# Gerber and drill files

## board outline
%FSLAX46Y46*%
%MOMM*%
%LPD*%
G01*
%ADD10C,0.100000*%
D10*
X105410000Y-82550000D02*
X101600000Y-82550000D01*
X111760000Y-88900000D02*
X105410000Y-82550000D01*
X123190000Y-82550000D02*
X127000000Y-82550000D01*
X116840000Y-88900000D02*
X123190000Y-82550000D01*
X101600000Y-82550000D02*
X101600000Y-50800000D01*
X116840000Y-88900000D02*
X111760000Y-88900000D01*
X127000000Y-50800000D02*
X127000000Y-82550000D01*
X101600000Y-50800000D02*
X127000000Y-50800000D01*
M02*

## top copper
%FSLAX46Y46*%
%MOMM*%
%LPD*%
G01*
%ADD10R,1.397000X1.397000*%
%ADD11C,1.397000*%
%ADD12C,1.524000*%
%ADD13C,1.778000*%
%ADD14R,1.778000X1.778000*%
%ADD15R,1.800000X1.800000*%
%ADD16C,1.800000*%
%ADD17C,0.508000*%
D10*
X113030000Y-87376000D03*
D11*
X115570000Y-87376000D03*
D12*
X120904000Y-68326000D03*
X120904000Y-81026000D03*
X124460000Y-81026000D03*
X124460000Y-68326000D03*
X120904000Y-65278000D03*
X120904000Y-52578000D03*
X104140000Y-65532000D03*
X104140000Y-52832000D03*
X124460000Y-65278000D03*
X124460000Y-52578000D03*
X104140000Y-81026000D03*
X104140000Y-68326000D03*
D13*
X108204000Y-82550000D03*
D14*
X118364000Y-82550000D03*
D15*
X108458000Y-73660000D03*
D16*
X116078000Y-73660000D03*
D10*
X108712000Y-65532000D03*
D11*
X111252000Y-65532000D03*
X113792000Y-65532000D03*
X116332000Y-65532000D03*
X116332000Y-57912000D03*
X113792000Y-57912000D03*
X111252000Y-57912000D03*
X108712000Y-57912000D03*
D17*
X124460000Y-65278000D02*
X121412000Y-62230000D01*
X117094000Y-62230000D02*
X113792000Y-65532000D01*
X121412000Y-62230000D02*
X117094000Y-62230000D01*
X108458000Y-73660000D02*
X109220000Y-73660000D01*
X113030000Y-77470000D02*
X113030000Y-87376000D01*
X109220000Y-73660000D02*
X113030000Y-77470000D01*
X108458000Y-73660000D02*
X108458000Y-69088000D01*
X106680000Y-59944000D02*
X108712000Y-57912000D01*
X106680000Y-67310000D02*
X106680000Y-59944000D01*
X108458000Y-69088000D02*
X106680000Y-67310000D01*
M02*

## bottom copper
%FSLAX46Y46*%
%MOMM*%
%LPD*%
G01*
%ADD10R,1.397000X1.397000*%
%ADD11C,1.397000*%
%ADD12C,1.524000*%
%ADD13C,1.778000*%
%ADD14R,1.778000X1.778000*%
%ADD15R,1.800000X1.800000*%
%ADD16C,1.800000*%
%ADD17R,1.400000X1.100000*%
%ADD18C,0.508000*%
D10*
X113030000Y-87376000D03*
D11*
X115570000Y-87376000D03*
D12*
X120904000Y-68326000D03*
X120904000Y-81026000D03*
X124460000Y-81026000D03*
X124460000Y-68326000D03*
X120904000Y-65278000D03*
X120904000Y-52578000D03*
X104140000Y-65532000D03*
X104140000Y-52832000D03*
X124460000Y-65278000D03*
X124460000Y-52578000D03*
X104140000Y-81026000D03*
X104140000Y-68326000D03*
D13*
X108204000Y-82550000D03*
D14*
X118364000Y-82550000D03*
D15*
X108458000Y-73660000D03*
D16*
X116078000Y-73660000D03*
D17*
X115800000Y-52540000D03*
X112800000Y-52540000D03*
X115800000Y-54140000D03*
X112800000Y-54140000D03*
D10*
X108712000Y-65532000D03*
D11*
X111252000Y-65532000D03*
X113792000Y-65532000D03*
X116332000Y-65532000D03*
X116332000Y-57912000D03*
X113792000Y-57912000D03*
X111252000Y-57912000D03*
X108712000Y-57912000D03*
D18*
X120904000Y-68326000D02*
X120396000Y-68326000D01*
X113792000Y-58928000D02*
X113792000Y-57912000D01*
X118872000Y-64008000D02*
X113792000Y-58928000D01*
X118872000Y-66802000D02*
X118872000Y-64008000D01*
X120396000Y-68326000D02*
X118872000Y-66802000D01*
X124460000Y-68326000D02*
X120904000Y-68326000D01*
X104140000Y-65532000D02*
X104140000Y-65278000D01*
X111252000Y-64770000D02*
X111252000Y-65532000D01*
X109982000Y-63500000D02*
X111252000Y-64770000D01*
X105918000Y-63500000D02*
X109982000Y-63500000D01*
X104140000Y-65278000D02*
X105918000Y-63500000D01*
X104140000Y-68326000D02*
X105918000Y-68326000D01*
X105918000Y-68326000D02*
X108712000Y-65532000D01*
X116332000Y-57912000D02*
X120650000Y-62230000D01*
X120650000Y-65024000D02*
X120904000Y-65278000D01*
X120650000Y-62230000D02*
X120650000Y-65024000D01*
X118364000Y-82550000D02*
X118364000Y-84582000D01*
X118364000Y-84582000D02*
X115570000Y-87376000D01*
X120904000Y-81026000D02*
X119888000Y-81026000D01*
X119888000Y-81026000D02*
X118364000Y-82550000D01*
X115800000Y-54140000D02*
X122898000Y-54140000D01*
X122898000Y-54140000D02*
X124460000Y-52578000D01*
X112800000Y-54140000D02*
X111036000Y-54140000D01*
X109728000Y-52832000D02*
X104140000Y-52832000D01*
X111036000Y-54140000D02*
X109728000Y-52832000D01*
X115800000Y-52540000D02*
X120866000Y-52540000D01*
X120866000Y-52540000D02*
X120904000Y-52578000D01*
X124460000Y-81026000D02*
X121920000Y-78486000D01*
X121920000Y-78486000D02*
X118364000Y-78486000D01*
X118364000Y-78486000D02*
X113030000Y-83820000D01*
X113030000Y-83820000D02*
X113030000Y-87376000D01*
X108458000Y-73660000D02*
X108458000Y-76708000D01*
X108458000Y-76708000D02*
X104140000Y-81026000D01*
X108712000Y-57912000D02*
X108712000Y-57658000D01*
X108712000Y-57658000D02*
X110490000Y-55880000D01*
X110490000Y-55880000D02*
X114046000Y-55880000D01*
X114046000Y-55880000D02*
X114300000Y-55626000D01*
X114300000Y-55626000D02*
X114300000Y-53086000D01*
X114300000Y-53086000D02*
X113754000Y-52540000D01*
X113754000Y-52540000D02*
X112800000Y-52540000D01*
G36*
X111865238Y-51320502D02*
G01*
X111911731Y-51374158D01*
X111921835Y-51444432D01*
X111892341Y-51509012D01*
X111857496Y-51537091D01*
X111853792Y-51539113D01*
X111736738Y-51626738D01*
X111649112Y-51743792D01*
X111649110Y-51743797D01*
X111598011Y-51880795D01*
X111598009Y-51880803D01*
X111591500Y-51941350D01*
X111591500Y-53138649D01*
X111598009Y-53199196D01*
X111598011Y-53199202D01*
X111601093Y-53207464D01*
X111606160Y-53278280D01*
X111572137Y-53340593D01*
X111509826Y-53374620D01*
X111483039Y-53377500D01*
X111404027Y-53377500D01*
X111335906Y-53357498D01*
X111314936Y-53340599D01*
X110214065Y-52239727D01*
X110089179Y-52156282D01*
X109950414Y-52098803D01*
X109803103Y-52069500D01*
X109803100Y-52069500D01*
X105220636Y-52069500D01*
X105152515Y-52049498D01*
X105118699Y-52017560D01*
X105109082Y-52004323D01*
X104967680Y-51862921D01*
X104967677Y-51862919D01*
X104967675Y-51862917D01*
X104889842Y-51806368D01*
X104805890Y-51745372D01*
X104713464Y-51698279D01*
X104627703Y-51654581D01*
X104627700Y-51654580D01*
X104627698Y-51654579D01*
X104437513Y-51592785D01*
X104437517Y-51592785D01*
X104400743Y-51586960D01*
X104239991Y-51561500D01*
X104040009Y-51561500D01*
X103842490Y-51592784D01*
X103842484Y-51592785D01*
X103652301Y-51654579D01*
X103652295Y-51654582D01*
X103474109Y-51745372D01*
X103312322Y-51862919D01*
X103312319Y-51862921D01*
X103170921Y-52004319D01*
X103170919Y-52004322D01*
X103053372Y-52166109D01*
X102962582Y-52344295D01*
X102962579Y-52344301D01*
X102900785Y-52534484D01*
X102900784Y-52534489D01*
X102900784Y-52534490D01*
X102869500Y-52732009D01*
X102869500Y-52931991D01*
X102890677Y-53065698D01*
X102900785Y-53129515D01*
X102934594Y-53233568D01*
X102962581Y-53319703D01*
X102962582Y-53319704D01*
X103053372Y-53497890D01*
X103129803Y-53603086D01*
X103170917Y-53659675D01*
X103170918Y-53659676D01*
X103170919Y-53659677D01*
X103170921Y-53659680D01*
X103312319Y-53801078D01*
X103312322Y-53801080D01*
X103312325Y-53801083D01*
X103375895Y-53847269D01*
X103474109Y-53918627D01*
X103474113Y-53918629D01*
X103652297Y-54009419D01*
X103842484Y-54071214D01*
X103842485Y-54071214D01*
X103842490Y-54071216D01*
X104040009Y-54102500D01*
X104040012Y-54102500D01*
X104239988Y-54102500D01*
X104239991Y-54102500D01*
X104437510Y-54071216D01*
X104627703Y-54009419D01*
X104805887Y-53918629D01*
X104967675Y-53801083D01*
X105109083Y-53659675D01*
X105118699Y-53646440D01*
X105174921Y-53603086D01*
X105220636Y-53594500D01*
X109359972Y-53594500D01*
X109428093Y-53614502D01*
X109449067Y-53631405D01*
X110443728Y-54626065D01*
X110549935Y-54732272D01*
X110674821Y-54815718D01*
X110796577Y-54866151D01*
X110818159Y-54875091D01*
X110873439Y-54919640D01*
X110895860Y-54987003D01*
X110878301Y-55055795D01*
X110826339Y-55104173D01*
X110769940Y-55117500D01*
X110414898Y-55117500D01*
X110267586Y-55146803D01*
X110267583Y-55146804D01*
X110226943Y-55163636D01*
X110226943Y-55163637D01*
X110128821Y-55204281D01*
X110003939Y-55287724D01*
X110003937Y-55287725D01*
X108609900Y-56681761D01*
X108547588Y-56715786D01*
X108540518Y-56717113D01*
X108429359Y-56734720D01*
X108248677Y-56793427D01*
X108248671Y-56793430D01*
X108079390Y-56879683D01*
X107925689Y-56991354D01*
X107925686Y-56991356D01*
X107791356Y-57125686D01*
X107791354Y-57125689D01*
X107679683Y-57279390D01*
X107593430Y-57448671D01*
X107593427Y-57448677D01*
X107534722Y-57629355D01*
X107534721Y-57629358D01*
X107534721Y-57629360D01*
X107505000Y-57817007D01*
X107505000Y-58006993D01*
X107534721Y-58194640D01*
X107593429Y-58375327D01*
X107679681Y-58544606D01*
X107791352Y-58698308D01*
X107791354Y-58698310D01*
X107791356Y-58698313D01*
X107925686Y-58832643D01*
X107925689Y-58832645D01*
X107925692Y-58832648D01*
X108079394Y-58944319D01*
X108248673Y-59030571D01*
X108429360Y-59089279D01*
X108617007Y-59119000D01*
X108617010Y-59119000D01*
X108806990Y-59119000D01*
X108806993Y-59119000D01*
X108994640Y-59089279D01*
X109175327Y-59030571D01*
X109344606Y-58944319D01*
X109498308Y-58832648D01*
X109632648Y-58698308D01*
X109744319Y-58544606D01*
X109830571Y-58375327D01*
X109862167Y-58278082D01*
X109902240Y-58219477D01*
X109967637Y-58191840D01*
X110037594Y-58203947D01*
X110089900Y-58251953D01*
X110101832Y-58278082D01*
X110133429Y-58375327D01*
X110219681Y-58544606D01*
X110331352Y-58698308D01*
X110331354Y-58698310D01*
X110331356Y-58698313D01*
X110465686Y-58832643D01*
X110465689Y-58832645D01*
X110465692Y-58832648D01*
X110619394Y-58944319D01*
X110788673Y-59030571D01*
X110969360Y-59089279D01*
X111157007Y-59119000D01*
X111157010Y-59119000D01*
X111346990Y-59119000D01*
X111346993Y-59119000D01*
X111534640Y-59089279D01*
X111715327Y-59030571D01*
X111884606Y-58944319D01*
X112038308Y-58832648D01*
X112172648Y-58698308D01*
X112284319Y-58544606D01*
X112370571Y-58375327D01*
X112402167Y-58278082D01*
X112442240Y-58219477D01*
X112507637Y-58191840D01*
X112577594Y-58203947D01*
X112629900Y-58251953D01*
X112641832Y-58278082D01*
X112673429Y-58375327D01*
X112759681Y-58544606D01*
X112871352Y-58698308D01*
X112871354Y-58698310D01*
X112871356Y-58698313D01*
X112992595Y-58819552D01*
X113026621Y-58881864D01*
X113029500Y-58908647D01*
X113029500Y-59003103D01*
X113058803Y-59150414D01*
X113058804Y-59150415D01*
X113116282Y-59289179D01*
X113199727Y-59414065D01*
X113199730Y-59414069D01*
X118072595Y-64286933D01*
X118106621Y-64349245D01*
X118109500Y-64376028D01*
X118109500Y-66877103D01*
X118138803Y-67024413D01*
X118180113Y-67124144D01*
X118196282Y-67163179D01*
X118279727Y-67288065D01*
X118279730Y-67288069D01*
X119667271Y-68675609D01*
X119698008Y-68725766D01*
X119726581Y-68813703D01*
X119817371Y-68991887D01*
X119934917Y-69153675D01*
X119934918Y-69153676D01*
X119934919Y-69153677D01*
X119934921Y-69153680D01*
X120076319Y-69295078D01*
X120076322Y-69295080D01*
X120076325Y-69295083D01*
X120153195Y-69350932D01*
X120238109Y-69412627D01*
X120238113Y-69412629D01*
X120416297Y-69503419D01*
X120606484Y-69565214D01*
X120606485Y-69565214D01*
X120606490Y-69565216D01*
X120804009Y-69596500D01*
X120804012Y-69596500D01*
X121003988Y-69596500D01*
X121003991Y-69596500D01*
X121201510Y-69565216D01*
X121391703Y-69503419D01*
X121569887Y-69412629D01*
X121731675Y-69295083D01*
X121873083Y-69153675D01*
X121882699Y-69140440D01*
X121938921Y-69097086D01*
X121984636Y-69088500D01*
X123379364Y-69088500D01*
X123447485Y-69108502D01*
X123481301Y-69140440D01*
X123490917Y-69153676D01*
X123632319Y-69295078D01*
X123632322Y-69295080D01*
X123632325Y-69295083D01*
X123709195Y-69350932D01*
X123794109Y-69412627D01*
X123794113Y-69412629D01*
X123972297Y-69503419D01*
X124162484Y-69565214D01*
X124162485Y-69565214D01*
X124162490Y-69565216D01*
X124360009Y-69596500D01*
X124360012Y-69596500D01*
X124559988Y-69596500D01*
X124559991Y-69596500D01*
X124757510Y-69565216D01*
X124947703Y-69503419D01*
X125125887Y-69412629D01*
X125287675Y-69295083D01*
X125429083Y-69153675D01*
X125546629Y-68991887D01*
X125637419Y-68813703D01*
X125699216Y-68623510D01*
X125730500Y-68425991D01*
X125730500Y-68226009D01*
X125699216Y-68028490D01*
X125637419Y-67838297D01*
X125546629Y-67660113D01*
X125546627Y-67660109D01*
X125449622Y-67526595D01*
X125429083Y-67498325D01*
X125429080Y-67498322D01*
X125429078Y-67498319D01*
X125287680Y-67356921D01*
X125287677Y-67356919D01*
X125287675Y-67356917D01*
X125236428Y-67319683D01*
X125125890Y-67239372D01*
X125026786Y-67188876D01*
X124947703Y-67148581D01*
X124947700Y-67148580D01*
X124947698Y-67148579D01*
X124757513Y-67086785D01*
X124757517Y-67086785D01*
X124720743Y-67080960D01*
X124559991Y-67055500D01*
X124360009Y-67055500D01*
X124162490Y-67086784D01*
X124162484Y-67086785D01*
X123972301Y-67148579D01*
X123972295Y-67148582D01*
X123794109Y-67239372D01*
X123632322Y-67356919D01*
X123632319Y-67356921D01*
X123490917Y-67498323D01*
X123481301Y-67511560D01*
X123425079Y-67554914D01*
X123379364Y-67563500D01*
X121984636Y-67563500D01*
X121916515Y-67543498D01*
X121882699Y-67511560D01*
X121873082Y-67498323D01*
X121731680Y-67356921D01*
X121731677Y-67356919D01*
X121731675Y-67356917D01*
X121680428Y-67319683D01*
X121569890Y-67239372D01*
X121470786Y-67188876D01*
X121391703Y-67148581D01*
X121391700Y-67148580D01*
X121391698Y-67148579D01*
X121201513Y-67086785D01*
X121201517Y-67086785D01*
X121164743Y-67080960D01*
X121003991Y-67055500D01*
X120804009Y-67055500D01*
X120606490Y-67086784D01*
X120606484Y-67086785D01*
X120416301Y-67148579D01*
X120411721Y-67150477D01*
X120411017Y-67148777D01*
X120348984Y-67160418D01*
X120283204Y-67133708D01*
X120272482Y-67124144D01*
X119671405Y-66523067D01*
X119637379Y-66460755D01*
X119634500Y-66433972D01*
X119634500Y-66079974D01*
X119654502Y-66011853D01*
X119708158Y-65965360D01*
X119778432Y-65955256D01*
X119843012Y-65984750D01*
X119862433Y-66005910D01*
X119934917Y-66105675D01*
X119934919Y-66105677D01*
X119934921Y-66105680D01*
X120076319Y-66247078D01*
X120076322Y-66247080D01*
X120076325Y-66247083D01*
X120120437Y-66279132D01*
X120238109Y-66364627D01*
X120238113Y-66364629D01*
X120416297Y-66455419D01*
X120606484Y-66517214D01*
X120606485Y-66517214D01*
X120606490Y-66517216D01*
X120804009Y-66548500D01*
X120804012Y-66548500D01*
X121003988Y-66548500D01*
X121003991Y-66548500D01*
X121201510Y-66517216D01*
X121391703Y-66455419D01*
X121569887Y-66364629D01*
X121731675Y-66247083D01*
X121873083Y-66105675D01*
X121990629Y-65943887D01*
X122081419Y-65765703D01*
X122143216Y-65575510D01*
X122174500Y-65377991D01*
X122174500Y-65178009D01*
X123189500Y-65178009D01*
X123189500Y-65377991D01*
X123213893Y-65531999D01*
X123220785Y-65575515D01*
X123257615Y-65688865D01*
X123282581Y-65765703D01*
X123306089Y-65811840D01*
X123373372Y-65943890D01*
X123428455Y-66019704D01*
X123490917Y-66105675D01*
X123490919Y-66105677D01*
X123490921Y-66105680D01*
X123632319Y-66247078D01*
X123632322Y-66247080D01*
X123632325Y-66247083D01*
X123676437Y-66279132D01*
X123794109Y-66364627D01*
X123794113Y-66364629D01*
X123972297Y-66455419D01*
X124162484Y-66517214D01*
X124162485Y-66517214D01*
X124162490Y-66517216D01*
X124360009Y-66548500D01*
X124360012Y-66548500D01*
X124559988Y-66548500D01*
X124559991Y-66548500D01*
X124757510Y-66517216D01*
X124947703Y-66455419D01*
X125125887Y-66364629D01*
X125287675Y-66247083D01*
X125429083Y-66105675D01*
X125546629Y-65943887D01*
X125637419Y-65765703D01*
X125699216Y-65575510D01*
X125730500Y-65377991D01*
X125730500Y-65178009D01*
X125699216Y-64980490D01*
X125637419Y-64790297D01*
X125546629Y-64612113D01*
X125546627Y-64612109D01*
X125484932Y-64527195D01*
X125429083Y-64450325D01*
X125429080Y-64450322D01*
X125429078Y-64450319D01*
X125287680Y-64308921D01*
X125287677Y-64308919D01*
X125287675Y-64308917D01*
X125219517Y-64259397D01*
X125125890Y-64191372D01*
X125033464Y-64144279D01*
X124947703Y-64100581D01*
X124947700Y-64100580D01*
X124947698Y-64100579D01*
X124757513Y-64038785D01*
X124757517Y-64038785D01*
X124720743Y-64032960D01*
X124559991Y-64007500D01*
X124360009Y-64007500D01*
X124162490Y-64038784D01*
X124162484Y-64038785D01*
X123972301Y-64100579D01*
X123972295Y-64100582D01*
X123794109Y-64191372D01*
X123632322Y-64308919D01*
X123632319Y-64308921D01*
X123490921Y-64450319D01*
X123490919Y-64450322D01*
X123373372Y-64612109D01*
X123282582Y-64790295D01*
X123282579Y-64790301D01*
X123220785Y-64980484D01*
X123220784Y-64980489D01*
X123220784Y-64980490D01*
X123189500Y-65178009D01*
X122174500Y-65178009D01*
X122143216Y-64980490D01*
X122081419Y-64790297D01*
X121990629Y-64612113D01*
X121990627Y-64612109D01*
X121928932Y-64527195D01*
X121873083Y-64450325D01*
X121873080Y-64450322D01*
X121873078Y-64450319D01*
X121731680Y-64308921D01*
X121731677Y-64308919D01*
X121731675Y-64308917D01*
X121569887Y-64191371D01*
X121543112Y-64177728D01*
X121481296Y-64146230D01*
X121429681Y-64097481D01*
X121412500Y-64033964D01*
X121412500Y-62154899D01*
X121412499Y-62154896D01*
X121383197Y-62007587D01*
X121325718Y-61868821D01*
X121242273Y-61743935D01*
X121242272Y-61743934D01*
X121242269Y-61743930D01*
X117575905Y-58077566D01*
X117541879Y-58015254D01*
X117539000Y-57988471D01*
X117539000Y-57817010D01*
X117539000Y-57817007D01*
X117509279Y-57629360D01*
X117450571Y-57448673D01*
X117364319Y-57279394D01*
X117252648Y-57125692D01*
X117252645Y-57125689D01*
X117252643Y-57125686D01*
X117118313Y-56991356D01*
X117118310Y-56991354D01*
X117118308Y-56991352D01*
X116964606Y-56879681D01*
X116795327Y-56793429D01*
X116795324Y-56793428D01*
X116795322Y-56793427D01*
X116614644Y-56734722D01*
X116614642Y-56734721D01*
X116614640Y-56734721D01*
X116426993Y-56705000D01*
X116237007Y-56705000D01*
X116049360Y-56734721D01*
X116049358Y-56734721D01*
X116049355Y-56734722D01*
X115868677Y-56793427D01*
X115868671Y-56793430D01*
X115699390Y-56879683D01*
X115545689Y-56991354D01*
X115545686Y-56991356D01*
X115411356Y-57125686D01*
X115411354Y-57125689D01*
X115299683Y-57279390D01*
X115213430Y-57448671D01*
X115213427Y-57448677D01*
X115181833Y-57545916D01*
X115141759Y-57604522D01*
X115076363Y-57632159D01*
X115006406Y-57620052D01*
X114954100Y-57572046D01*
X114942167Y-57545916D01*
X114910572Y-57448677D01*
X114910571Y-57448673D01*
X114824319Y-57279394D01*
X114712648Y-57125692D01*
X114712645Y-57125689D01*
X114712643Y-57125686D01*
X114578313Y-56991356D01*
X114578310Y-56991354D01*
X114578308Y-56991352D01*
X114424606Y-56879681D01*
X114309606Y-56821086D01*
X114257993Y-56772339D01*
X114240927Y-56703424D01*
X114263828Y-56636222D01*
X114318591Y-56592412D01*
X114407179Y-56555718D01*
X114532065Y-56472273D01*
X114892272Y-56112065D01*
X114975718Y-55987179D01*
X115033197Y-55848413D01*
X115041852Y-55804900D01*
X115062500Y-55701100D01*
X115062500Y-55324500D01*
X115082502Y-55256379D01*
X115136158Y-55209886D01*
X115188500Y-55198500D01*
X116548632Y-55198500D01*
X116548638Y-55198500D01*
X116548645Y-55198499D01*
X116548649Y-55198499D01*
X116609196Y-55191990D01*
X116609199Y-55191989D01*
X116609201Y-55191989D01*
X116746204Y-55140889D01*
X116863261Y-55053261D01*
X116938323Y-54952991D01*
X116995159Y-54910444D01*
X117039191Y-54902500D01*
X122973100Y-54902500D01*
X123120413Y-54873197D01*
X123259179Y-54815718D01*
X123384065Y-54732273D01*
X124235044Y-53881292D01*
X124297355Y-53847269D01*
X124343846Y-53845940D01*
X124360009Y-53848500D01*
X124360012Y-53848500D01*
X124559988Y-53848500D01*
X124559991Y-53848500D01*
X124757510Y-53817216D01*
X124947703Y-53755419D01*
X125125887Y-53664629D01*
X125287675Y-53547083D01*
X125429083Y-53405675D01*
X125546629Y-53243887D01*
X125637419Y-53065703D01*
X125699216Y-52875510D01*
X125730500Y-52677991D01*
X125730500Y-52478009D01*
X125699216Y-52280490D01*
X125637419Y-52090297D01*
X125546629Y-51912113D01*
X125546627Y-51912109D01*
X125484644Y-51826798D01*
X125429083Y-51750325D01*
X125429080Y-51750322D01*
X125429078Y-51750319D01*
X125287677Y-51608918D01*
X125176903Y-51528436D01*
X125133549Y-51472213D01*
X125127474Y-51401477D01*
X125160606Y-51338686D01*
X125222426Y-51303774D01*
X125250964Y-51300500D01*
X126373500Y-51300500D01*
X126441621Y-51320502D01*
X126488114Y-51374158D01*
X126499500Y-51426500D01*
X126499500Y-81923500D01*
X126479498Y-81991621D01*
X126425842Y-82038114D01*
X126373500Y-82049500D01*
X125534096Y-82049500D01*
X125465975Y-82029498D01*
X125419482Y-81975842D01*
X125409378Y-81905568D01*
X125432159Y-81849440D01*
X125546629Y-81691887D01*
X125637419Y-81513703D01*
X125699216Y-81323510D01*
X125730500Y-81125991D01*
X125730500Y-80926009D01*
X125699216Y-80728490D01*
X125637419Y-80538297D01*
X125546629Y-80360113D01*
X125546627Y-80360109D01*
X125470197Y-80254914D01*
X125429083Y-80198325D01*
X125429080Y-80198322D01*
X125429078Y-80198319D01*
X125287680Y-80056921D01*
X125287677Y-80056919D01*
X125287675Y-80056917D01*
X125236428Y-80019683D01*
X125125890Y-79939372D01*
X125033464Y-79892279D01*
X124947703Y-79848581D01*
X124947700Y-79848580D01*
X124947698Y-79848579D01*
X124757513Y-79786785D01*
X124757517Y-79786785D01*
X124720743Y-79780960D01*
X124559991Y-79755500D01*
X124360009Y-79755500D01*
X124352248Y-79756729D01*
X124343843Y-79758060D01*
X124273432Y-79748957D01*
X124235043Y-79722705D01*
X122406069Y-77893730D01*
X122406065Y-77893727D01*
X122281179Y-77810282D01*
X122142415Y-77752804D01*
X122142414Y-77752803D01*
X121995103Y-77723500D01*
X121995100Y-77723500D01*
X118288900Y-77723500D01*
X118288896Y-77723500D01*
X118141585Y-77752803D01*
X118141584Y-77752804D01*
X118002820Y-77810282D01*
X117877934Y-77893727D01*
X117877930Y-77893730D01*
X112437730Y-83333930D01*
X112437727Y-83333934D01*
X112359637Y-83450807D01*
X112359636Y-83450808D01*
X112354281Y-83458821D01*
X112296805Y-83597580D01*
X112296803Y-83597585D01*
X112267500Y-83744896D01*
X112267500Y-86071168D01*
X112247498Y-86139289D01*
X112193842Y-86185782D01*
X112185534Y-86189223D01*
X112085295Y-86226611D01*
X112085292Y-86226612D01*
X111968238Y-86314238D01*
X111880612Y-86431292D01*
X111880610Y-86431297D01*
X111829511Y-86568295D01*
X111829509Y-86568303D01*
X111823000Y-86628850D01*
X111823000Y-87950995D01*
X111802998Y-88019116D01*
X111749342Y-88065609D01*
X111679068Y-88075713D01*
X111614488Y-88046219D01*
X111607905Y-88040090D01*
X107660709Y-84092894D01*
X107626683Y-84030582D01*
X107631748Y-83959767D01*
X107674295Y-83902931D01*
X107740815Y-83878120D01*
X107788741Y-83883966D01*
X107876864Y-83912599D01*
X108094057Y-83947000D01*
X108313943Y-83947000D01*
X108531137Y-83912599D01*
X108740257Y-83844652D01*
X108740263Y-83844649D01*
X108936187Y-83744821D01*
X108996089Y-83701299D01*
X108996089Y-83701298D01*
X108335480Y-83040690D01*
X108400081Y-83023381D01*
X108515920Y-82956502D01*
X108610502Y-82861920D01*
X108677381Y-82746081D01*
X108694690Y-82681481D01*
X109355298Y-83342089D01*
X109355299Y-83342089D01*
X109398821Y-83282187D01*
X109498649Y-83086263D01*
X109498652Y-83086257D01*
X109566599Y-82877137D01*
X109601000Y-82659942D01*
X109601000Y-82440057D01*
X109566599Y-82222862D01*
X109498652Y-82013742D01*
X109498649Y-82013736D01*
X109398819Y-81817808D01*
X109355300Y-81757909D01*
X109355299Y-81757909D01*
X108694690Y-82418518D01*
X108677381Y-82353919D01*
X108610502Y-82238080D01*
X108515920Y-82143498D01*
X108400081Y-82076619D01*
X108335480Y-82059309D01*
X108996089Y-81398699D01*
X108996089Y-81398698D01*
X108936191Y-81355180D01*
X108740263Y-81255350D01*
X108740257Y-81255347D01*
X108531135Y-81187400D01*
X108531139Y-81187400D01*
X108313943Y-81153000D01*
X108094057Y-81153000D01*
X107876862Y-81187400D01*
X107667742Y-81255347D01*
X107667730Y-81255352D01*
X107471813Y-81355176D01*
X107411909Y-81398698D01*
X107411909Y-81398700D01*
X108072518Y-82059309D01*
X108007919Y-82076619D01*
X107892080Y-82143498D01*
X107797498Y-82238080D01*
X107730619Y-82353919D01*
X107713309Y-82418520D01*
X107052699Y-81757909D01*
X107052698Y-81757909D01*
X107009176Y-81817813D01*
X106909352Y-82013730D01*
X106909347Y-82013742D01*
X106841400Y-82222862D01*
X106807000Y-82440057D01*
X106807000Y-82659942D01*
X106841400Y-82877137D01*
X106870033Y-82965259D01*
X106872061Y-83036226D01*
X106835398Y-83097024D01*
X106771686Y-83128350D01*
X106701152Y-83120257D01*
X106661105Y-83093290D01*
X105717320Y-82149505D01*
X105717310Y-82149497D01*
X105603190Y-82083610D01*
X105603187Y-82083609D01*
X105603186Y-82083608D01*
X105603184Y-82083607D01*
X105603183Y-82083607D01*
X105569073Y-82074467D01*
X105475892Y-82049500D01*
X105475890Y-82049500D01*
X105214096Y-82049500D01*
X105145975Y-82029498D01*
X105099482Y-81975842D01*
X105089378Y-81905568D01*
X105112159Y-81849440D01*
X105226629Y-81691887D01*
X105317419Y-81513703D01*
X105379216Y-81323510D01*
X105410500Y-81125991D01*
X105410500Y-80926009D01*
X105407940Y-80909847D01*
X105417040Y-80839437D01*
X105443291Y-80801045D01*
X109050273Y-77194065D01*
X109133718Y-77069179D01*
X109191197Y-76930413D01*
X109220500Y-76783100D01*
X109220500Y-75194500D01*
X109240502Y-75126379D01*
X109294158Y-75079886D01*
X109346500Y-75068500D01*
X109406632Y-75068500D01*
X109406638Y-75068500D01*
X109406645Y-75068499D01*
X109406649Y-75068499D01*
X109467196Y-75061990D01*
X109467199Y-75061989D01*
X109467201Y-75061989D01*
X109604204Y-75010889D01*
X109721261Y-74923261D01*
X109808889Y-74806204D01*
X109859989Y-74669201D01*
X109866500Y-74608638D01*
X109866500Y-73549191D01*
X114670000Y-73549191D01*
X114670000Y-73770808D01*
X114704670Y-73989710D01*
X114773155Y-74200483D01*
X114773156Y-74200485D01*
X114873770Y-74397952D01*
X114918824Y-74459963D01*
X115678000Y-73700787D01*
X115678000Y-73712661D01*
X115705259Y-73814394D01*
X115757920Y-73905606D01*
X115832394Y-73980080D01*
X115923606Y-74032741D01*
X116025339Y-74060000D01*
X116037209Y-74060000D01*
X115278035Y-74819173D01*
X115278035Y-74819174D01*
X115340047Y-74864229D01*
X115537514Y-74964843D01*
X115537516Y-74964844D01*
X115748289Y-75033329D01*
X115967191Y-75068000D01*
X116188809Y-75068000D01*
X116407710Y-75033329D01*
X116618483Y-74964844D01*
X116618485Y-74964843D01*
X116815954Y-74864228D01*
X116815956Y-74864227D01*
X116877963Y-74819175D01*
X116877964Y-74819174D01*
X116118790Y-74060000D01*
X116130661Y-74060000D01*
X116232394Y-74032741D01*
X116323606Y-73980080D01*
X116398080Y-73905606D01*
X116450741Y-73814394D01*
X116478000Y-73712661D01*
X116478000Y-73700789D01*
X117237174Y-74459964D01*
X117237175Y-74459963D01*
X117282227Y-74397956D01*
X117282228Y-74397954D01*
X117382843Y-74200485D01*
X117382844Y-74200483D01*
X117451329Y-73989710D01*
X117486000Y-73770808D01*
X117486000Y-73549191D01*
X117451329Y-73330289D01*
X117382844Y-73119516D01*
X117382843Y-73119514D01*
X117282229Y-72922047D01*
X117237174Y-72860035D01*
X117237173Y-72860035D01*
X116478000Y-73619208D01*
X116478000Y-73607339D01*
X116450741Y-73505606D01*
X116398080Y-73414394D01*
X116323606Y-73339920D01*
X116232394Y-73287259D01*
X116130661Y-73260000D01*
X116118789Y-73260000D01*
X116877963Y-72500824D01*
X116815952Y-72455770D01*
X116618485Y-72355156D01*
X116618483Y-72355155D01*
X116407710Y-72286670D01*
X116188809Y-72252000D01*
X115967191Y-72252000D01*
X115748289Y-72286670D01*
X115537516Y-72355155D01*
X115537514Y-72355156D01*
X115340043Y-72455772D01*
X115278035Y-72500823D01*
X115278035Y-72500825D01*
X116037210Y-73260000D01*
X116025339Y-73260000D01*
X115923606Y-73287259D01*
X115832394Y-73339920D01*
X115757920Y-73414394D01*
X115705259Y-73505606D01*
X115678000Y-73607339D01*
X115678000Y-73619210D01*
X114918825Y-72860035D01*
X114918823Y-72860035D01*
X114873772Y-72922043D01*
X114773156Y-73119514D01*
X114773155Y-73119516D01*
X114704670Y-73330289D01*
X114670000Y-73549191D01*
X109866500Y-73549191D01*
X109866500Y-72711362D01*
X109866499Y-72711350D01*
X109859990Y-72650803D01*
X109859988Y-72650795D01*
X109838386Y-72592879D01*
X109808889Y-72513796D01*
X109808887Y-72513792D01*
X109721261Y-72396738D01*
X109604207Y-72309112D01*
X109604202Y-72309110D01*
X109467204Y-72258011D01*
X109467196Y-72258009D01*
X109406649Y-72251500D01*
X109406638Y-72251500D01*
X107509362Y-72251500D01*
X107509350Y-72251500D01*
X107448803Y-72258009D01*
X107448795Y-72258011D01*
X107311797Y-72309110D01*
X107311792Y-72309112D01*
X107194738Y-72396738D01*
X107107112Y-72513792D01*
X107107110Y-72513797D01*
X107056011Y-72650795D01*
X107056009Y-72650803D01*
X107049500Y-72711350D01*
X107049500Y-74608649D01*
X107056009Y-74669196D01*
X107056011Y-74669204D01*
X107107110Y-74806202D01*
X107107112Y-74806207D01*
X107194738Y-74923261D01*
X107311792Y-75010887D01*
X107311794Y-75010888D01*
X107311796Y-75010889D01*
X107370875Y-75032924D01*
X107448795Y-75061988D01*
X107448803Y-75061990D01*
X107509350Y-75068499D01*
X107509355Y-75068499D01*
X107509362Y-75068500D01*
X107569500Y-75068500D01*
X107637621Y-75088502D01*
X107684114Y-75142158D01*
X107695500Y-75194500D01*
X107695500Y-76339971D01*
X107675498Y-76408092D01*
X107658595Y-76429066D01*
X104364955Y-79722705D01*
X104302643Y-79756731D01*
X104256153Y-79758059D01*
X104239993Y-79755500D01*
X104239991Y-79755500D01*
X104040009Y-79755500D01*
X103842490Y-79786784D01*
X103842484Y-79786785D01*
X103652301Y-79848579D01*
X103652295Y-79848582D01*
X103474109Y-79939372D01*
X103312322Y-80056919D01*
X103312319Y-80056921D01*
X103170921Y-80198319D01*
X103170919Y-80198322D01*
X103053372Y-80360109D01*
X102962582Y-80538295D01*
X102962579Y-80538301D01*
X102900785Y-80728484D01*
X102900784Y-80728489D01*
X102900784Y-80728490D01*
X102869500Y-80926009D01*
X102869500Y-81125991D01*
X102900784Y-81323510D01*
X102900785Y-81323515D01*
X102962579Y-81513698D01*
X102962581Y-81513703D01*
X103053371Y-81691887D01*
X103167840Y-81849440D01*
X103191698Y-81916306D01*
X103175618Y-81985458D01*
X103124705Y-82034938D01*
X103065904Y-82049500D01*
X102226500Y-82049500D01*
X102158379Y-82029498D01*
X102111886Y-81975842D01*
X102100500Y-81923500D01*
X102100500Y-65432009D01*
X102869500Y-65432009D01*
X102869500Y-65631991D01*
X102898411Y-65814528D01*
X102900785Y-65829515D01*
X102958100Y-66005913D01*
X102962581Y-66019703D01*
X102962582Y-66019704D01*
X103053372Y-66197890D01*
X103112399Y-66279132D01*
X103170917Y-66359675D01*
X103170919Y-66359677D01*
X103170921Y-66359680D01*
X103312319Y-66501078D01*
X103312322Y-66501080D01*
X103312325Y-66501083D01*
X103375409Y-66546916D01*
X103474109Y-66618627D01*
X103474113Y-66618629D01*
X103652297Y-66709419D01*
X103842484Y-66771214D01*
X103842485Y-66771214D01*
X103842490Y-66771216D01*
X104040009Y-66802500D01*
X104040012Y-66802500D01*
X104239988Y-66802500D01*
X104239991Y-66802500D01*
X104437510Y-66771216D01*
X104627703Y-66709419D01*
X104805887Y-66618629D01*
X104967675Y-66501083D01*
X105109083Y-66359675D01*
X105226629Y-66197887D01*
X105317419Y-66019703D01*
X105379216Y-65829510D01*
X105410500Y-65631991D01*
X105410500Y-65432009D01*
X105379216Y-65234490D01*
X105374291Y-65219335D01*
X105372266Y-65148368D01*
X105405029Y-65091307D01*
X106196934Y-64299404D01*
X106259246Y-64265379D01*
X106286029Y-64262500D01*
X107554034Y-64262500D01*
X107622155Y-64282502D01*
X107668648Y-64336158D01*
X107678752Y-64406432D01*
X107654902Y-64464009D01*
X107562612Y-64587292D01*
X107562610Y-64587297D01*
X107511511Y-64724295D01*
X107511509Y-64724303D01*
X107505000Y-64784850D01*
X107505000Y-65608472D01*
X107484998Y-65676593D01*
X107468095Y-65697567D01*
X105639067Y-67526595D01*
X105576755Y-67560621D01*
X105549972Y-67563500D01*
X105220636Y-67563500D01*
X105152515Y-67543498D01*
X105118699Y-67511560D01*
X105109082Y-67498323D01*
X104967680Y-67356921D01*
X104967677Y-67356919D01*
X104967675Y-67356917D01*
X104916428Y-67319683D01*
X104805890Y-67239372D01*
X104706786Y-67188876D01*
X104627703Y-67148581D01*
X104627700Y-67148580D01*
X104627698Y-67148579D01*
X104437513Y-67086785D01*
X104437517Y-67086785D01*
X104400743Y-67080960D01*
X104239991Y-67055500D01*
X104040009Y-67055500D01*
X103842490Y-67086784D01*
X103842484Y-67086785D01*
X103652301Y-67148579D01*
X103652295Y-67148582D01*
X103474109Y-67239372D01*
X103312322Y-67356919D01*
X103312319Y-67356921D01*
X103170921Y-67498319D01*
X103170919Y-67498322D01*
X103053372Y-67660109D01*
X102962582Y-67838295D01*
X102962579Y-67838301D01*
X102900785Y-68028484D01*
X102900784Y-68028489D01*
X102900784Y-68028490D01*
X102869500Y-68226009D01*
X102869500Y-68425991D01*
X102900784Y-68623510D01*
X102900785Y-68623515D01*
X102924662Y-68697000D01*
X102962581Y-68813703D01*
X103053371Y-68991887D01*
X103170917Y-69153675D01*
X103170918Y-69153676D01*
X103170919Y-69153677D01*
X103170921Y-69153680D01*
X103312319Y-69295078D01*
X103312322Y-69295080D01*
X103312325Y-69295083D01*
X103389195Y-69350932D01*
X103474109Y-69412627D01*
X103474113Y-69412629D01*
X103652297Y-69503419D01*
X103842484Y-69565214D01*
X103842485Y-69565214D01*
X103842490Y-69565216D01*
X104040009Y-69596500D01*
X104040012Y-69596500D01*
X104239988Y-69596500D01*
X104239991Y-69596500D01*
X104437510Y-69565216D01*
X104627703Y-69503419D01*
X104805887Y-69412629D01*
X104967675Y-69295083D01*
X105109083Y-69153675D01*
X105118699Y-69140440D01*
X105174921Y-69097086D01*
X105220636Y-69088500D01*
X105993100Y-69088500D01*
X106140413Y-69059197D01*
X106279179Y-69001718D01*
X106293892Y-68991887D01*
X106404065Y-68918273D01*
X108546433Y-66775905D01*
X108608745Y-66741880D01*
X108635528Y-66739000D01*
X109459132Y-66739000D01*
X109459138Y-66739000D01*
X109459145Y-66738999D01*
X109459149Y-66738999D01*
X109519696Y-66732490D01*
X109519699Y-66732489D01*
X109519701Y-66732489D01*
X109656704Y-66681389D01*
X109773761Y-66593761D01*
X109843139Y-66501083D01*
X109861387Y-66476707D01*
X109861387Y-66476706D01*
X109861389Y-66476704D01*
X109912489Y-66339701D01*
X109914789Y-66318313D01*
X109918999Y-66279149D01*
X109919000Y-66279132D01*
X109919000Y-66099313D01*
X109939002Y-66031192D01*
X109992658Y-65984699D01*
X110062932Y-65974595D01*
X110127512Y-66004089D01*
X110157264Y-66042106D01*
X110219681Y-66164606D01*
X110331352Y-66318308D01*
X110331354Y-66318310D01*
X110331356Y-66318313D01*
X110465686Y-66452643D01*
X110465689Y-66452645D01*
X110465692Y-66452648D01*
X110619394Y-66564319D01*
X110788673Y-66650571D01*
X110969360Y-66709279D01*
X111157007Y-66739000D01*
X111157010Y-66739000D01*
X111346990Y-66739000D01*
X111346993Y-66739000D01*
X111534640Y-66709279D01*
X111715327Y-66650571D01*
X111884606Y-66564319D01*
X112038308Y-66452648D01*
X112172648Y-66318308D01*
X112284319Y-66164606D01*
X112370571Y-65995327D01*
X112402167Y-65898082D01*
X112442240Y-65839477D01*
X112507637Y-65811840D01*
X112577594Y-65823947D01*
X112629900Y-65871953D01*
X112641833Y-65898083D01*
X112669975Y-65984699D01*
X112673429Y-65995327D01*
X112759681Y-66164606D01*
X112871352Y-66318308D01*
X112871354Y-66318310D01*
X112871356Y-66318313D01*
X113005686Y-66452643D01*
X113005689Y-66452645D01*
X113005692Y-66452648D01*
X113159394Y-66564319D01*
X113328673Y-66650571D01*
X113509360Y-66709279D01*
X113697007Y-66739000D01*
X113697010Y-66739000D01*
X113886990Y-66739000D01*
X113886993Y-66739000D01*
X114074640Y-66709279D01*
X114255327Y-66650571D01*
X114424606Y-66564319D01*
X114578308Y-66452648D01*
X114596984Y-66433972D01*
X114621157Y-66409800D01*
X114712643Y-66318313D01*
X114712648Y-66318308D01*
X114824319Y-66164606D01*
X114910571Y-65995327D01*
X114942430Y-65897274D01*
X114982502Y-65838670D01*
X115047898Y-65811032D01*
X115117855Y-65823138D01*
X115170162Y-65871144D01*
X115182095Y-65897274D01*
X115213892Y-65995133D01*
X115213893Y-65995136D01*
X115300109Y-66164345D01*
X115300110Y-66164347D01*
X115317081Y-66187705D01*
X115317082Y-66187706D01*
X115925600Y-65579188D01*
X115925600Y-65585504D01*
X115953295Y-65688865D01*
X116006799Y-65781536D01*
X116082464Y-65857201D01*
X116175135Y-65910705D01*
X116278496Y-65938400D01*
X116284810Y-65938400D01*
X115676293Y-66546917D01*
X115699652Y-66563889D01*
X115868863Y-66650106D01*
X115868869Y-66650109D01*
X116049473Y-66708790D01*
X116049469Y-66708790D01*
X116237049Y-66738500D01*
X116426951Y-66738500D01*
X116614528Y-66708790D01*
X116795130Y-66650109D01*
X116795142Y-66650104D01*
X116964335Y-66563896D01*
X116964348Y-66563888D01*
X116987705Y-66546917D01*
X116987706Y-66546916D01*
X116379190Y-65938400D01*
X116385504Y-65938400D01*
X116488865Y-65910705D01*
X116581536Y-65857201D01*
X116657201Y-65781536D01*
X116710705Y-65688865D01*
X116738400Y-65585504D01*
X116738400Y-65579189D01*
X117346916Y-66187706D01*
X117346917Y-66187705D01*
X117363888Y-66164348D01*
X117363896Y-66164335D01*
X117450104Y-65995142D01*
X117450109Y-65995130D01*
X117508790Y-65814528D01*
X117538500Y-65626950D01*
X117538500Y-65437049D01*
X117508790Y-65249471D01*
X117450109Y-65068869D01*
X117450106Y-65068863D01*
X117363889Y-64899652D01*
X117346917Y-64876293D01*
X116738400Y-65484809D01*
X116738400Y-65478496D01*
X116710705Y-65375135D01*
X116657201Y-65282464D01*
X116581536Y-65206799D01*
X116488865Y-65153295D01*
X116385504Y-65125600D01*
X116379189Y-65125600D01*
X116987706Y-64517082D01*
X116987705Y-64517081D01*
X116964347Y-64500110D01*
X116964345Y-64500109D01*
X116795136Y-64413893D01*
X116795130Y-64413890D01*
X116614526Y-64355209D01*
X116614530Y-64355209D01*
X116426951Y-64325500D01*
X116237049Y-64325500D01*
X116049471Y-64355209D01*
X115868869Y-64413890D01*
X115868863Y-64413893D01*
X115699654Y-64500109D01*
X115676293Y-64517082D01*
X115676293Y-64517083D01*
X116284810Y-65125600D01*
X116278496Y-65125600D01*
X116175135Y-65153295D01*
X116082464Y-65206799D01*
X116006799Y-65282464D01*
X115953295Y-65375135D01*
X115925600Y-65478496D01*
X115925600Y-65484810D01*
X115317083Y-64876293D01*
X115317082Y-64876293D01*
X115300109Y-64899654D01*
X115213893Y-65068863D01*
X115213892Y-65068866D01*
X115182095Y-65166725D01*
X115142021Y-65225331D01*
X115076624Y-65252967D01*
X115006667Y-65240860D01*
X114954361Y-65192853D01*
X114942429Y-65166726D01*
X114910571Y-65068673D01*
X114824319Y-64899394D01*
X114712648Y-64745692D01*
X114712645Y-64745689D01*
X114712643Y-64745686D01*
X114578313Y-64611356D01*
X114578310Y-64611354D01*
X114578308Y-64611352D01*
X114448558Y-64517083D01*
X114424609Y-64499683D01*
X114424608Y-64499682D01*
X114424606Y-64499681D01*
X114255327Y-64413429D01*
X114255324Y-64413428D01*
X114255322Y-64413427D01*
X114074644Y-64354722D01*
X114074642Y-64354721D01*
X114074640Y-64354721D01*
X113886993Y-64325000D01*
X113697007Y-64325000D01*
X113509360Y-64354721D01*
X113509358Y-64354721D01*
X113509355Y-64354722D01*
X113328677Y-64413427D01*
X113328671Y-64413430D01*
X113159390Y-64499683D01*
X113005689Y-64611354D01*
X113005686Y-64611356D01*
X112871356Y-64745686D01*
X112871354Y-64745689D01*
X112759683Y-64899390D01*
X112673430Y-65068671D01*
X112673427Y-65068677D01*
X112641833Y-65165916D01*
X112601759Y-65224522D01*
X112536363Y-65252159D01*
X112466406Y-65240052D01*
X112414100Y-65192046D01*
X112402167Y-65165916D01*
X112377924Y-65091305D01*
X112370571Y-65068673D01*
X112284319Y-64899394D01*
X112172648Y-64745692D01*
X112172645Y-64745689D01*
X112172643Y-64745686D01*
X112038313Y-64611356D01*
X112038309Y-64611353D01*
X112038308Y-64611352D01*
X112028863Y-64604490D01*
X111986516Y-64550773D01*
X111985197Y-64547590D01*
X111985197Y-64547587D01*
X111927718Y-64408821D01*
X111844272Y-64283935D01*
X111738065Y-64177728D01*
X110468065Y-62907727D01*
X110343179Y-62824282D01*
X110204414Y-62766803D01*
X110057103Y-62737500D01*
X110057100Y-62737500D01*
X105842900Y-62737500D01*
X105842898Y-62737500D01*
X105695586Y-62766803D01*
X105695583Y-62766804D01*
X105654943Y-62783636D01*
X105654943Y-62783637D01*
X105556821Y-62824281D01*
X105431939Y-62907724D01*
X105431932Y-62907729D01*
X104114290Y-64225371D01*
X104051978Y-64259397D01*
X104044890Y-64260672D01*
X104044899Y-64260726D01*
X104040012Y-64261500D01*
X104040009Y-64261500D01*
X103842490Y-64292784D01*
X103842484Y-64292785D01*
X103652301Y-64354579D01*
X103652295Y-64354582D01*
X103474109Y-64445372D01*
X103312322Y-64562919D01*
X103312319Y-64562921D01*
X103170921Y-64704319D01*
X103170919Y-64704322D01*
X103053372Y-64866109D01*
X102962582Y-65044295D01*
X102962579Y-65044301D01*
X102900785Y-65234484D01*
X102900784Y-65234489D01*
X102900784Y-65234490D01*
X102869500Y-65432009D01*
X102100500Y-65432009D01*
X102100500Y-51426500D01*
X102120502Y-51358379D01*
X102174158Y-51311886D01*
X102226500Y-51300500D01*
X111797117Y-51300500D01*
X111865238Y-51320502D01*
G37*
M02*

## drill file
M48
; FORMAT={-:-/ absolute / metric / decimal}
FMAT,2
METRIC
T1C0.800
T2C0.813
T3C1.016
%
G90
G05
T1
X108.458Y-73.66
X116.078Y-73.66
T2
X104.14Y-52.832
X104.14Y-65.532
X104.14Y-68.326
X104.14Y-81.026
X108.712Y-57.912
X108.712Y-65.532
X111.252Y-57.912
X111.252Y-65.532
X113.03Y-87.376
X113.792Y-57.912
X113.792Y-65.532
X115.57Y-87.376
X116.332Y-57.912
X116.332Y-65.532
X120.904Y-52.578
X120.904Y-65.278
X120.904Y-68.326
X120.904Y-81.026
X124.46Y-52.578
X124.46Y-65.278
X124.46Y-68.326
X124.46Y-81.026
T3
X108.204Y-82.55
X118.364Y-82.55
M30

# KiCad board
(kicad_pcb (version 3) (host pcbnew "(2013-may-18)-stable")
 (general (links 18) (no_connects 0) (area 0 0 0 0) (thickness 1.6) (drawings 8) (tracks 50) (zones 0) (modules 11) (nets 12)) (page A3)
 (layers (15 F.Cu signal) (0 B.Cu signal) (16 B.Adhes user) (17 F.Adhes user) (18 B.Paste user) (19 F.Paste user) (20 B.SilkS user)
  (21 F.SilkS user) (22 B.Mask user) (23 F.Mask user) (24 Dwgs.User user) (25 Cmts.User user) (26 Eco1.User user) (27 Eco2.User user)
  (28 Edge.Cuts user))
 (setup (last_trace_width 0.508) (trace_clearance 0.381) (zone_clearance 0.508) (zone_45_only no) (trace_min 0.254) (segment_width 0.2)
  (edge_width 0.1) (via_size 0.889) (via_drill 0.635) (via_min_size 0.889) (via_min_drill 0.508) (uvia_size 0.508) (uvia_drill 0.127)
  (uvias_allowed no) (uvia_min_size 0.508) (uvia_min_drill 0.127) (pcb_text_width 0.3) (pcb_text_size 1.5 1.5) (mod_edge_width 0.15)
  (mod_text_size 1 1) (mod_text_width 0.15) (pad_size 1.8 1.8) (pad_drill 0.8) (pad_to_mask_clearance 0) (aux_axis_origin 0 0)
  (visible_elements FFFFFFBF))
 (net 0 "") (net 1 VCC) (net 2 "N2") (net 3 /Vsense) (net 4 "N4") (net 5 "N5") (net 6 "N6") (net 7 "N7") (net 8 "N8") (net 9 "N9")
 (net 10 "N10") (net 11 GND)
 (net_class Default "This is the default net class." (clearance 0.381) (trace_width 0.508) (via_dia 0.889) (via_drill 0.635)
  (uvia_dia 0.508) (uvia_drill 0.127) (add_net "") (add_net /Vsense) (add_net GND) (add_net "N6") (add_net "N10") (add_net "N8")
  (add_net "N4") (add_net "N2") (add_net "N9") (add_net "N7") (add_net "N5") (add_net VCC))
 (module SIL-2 (layer F.Cu) (at 114.3 87.376)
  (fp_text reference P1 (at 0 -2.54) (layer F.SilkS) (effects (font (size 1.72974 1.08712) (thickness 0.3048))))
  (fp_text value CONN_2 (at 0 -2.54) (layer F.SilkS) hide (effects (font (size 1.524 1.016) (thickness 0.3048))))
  (pad 1 thru_hole rect (at -1.27 0) (size 1.397 1.397) (drill 0.8128) (layers *.Cu *.Mask F.SilkS) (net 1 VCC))
  (pad 2 thru_hole circle (at 1.27 0) (size 1.397 1.397) (drill 0.8128) (layers *.Cu *.Mask F.SilkS) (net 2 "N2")))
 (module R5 (layer F.Cu) (at 120.904 74.676 270) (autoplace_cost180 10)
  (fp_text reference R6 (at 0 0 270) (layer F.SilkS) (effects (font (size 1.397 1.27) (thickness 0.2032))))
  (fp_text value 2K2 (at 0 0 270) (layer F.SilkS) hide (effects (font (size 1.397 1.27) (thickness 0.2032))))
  (pad 1 thru_hole circle (at -6.35 0 270) (size 1.524 1.524) (drill 0.8128) (layers *.Cu *.Mask F.SilkS) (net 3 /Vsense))
  (pad 2 thru_hole circle (at 6.35 0 270) (size 1.524 1.524) (drill 0.8128) (layers *.Cu *.Mask F.SilkS) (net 2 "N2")))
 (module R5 (layer F.Cu) (at 124.46 74.676 90) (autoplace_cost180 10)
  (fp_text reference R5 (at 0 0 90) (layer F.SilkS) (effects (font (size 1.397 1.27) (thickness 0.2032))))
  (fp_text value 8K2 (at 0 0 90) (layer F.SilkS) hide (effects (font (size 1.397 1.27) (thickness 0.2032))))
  (pad 1 thru_hole circle (at -6.35 0 90) (size 1.524 1.524) (drill 0.8128) (layers *.Cu *.Mask F.SilkS) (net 1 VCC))
  (pad 2 thru_hole circle (at 6.35 0 90) (size 1.524 1.524) (drill 0.8128) (layers *.Cu *.Mask F.SilkS) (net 3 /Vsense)))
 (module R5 (layer F.Cu) (at 120.904 58.928 90) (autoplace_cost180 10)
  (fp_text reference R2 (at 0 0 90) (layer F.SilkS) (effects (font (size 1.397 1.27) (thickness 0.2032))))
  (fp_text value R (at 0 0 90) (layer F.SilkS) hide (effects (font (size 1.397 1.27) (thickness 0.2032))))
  (pad 1 thru_hole circle (at -6.35 0 90) (size 1.524 1.524) (drill 0.8128) (layers *.Cu *.Mask F.SilkS) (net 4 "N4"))
  (pad 2 thru_hole circle (at 6.35 0 90) (size 1.524 1.524) (drill 0.8128) (layers *.Cu *.Mask F.SilkS) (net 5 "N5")))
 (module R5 (layer F.Cu) (at 104.14 59.182 90) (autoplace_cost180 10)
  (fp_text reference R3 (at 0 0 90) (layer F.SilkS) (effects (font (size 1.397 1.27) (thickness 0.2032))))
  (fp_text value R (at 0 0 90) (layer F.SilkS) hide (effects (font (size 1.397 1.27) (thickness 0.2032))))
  (pad 1 thru_hole circle (at -6.35 0 90) (size 1.524 1.524) (drill 0.8128) (layers *.Cu *.Mask F.SilkS) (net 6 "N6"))
  (pad 2 thru_hole circle (at 6.35 0 90) (size 1.524 1.524) (drill 0.8128) (layers *.Cu *.Mask F.SilkS) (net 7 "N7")))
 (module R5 (layer F.Cu) (at 124.46 58.928 90) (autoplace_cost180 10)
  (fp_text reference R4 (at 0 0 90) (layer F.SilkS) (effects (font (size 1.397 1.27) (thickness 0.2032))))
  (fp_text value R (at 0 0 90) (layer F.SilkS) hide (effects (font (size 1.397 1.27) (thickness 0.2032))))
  (pad 1 thru_hole circle (at -6.35 0 90) (size 1.524 1.524) (drill 0.8128) (layers *.Cu *.Mask F.SilkS) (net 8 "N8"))
  (pad 2 thru_hole circle (at 6.35 0 90) (size 1.524 1.524) (drill 0.8128) (layers *.Cu *.Mask F.SilkS) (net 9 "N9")))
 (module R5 (layer F.Cu) (at 104.14 74.676 90) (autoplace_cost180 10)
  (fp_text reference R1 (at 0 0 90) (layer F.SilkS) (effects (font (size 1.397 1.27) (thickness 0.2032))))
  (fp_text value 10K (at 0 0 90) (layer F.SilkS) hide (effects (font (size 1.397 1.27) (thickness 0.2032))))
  (pad 1 thru_hole circle (at -6.35 0 90) (size 1.524 1.524) (drill 0.8128) (layers *.Cu *.Mask F.SilkS) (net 1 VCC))
  (pad 2 thru_hole circle (at 6.35 0 90) (size 1.524 1.524) (drill 0.8128) (layers *.Cu *.Mask F.SilkS) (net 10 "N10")))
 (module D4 (layer F.Cu) (at 113.284 82.55)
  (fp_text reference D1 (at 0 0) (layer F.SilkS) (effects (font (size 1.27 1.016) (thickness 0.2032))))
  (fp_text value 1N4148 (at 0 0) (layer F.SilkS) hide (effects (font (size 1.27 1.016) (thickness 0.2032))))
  (pad 1 thru_hole circle (at -5.08 0) (size 1.778 1.778) (drill 1.016) (layers *.Cu *.Mask F.SilkS) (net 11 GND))
  (pad 2 thru_hole rect (at 5.08 0) (size 1.778 1.778) (drill 1.016) (layers *.Cu *.Mask F.SilkS) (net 2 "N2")))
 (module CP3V (layer F.Cu) (at 112.268 73.66)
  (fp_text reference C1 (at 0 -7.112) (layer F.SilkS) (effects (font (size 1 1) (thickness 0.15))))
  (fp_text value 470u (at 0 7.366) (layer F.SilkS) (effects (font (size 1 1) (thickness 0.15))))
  (pad 1 thru_hole rect (at -3.81 0) (size 1.8 1.8) (drill 0.8) (layers *.Cu *.Mask F.SilkS) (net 1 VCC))
  (pad 2 thru_hole circle (at 3.81 0) (size 1.8 1.8) (drill 0.8) (layers *.Cu *.Mask F.SilkS) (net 11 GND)))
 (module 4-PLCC (layer B.Cu) (at 114.3 53.34 180)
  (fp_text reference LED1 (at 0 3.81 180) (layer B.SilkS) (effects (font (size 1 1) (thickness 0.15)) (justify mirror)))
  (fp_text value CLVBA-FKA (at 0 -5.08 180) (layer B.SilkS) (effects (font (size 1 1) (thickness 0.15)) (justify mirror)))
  (pad 1 smd rect (at -1.5 0.8 180) (size 1.4 1.1) (layers B.Cu B.Paste B.Mask) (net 5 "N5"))
  (pad 2 smd rect (at 1.5 0.8 180) (size 1.4 1.1) (layers B.Cu B.Paste B.Mask) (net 1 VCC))
  (pad 3 smd rect (at -1.5 -0.8 180) (size 1.4 1.1) (layers B.Cu B.Paste B.Mask) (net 9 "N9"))
  (pad 4 smd rect (at 1.5 -0.8 180) (size 1.4 1.1) (layers B.Cu B.Paste B.Mask) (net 7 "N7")))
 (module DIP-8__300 (layer F.Cu) (at 112.522 61.722)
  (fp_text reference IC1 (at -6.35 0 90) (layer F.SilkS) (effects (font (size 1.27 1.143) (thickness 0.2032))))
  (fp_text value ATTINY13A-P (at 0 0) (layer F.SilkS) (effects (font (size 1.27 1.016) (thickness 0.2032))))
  (pad 1 thru_hole rect (at -3.81 3.81) (size 1.397 1.397) (drill 0.8128) (layers *.Cu *.Mask F.SilkS) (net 10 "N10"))
  (pad 2 thru_hole circle (at -1.27 3.81) (size 1.397 1.397) (drill 0.8128) (layers *.Cu *.Mask F.SilkS) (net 6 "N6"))
  (pad 3 thru_hole circle (at 1.27 3.81) (size 1.397 1.397) (drill 0.8128) (layers *.Cu *.Mask F.SilkS) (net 8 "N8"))
  (pad 4 thru_hole circle (at 3.81 3.81) (size 1.397 1.397) (drill 0.8128) (layers *.Cu *.Mask F.SilkS) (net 11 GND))
  (pad 5 thru_hole circle (at 3.81 -3.81) (size 1.397 1.397) (drill 0.8128) (layers *.Cu *.Mask F.SilkS) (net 4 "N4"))
  (pad 6 thru_hole circle (at 1.27 -3.81) (size 1.397 1.397) (drill 0.8128) (layers *.Cu *.Mask F.SilkS) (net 3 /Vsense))
  (pad 7 thru_hole circle (at -1.27 -3.81) (size 1.397 1.397) (drill 0.8128) (layers *.Cu *.Mask F.SilkS))
  (pad 8 thru_hole circle (at -3.81 -3.81) (size 1.397 1.397) (drill 0.8128) (layers *.Cu *.Mask F.SilkS) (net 1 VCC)))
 (gr_line (start 105.41 82.55) (end 101.6 82.55) (angle 90) (layer Edge.Cuts) (width 0.1))
 (gr_line (start 111.76 88.9) (end 105.41 82.55) (angle 90) (layer Edge.Cuts) (width 0.1))
 (gr_line (start 123.19 82.55) (end 127 82.55) (angle 90) (layer Edge.Cuts) (width 0.1))
 (gr_line (start 116.84 88.9) (end 123.19 82.55) (angle 90) (layer Edge.Cuts) (width 0.1))
 (gr_line (start 101.6 82.55) (end 101.6 50.8) (angle 90) (layer Edge.Cuts) (width 0.1))
 (gr_line (start 116.84 88.9) (end 111.76 88.9) (angle 90) (layer Edge.Cuts) (width 0.1))
 (gr_line (start 127 50.8) (end 127 82.55) (angle 90) (layer Edge.Cuts) (width 0.1))
 (gr_line (start 101.6 50.8) (end 127 50.8) (angle 90) (layer Edge.Cuts) (width 0.1))
 (segment (start 120.904 68.326) (end 120.396 68.326) (width 0.508) (layer B.Cu) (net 3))
 (segment (start 113.792 58.928) (end 113.792 57.912) (width 0.508) (layer B.Cu) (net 3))
 (segment (start 118.872 64.008) (end 113.792 58.928) (width 0.508) (layer B.Cu) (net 3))
 (segment (start 118.872 66.802) (end 118.872 64.008) (width 0.508) (layer B.Cu) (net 3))
 (segment (start 120.396 68.326) (end 118.872 66.802) (width 0.508) (layer B.Cu) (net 3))
 (segment (start 124.46 68.326) (end 120.904 68.326) (width 0.508) (layer B.Cu) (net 3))
 (segment (start 104.14 65.532) (end 104.14 65.278) (width 0.508) (layer B.Cu) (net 6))
 (segment (start 111.252 64.77) (end 111.252 65.532) (width 0.508) (layer B.Cu) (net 6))
 (segment (start 109.982 63.5) (end 111.252 64.77) (width 0.508) (layer B.Cu) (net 6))
 (segment (start 105.918 63.5) (end 109.982 63.5) (width 0.508) (layer B.Cu) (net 6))
 (segment (start 104.14 65.278) (end 105.918 63.5) (width 0.508) (layer B.Cu) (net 6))
 (segment (start 104.14 68.326) (end 105.918 68.326) (width 0.508) (layer B.Cu) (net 10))
 (segment (start 105.918 68.326) (end 108.712 65.532) (width 0.508) (layer B.Cu) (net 10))
 (segment (start 124.46 65.278) (end 121.412 62.23) (width 0.508) (layer F.Cu) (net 8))
 (segment (start 117.094 62.23) (end 113.792 65.532) (width 0.508) (layer F.Cu) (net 8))
 (segment (start 121.412 62.23) (end 117.094 62.23) (width 0.508) (layer F.Cu) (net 8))
 (segment (start 116.332 57.912) (end 120.65 62.23) (width 0.508) (layer B.Cu) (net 4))
 (segment (start 120.65 65.024) (end 120.904 65.278) (width 0.508) (layer B.Cu) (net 4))
 (segment (start 120.65 62.23) (end 120.65 65.024) (width 0.508) (layer B.Cu) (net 4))
 (segment (start 118.364 82.55) (end 118.364 84.582) (width 0.508) (layer B.Cu) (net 2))
 (segment (start 118.364 84.582) (end 115.57 87.376) (width 0.508) (layer B.Cu) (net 2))
 (segment (start 120.904 81.026) (end 119.888 81.026) (width 0.508) (layer B.Cu) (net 2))
 (segment (start 119.888 81.026) (end 118.364 82.55) (width 0.508) (layer B.Cu) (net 2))
 (segment (start 115.8 54.14) (end 122.898 54.14) (width 0.508) (layer B.Cu) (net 9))
 (segment (start 122.898 54.14) (end 124.46 52.578) (width 0.508) (layer B.Cu) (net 9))
 (segment (start 112.8 54.14) (end 111.036 54.14) (width 0.508) (layer B.Cu) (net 7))
 (segment (start 109.728 52.832) (end 104.14 52.832) (width 0.508) (layer B.Cu) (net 7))
 (segment (start 111.036 54.14) (end 109.728 52.832) (width 0.508) (layer B.Cu) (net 7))
 (segment (start 115.8 52.54) (end 120.866 52.54) (width 0.508) (layer B.Cu) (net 5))
 (segment (start 120.866 52.54) (end 120.904 52.578) (width 0.508) (layer B.Cu) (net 5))
 (segment (start 108.458 73.66) (end 109.22 73.66) (width 0.508) (layer F.Cu) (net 1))
 (segment (start 113.03 77.47) (end 113.03 87.376) (width 0.508) (layer F.Cu) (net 1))
 (segment (start 109.22 73.66) (end 113.03 77.47) (width 0.508) (layer F.Cu) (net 1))
 (segment (start 108.458 73.66) (end 108.458 69.088) (width 0.508) (layer F.Cu) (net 1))
 (segment (start 106.68 59.944) (end 108.712 57.912) (width 0.508) (layer F.Cu) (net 1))
 (segment (start 106.68 67.31) (end 106.68 59.944) (width 0.508) (layer F.Cu) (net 1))
 (segment (start 108.458 69.088) (end 106.68 67.31) (width 0.508) (layer F.Cu) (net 1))
 (segment (start 124.46 81.026) (end 121.92 78.486) (width 0.508) (layer B.Cu) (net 1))
 (segment (start 121.92 78.486) (end 118.364 78.486) (width 0.508) (layer B.Cu) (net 1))
 (segment (start 118.364 78.486) (end 113.03 83.82) (width 0.508) (layer B.Cu) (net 1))
 (segment (start 113.03 83.82) (end 113.03 87.376) (width 0.508) (layer B.Cu) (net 1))
 (segment (start 108.458 73.66) (end 108.458 76.708) (width 0.508) (layer B.Cu) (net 1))
 (segment (start 108.458 76.708) (end 104.14 81.026) (width 0.508) (layer B.Cu) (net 1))
 (segment (start 108.712 57.912) (end 108.712 57.658) (width 0.508) (layer B.Cu) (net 1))
 (segment (start 108.712 57.658) (end 110.49 55.88) (width 0.508) (layer B.Cu) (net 1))
 (segment (start 110.49 55.88) (end 114.046 55.88) (width 0.508) (layer B.Cu) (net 1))
 (segment (start 114.046 55.88) (end 114.3 55.626) (width 0.508) (layer B.Cu) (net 1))
 (segment (start 114.3 55.626) (end 114.3 53.086) (width 0.508) (layer B.Cu) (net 1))
 (segment (start 114.3 53.086) (end 113.754 52.54) (width 0.508) (layer B.Cu) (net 1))
 (segment (start 113.754 52.54) (end 112.8 52.54) (width 0.508) (layer B.Cu) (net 1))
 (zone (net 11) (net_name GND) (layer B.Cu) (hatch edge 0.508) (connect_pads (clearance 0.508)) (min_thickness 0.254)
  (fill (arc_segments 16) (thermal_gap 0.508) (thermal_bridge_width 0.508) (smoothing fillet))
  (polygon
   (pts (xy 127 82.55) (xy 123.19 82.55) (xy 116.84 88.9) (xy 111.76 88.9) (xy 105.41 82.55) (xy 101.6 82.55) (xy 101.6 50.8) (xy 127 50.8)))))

